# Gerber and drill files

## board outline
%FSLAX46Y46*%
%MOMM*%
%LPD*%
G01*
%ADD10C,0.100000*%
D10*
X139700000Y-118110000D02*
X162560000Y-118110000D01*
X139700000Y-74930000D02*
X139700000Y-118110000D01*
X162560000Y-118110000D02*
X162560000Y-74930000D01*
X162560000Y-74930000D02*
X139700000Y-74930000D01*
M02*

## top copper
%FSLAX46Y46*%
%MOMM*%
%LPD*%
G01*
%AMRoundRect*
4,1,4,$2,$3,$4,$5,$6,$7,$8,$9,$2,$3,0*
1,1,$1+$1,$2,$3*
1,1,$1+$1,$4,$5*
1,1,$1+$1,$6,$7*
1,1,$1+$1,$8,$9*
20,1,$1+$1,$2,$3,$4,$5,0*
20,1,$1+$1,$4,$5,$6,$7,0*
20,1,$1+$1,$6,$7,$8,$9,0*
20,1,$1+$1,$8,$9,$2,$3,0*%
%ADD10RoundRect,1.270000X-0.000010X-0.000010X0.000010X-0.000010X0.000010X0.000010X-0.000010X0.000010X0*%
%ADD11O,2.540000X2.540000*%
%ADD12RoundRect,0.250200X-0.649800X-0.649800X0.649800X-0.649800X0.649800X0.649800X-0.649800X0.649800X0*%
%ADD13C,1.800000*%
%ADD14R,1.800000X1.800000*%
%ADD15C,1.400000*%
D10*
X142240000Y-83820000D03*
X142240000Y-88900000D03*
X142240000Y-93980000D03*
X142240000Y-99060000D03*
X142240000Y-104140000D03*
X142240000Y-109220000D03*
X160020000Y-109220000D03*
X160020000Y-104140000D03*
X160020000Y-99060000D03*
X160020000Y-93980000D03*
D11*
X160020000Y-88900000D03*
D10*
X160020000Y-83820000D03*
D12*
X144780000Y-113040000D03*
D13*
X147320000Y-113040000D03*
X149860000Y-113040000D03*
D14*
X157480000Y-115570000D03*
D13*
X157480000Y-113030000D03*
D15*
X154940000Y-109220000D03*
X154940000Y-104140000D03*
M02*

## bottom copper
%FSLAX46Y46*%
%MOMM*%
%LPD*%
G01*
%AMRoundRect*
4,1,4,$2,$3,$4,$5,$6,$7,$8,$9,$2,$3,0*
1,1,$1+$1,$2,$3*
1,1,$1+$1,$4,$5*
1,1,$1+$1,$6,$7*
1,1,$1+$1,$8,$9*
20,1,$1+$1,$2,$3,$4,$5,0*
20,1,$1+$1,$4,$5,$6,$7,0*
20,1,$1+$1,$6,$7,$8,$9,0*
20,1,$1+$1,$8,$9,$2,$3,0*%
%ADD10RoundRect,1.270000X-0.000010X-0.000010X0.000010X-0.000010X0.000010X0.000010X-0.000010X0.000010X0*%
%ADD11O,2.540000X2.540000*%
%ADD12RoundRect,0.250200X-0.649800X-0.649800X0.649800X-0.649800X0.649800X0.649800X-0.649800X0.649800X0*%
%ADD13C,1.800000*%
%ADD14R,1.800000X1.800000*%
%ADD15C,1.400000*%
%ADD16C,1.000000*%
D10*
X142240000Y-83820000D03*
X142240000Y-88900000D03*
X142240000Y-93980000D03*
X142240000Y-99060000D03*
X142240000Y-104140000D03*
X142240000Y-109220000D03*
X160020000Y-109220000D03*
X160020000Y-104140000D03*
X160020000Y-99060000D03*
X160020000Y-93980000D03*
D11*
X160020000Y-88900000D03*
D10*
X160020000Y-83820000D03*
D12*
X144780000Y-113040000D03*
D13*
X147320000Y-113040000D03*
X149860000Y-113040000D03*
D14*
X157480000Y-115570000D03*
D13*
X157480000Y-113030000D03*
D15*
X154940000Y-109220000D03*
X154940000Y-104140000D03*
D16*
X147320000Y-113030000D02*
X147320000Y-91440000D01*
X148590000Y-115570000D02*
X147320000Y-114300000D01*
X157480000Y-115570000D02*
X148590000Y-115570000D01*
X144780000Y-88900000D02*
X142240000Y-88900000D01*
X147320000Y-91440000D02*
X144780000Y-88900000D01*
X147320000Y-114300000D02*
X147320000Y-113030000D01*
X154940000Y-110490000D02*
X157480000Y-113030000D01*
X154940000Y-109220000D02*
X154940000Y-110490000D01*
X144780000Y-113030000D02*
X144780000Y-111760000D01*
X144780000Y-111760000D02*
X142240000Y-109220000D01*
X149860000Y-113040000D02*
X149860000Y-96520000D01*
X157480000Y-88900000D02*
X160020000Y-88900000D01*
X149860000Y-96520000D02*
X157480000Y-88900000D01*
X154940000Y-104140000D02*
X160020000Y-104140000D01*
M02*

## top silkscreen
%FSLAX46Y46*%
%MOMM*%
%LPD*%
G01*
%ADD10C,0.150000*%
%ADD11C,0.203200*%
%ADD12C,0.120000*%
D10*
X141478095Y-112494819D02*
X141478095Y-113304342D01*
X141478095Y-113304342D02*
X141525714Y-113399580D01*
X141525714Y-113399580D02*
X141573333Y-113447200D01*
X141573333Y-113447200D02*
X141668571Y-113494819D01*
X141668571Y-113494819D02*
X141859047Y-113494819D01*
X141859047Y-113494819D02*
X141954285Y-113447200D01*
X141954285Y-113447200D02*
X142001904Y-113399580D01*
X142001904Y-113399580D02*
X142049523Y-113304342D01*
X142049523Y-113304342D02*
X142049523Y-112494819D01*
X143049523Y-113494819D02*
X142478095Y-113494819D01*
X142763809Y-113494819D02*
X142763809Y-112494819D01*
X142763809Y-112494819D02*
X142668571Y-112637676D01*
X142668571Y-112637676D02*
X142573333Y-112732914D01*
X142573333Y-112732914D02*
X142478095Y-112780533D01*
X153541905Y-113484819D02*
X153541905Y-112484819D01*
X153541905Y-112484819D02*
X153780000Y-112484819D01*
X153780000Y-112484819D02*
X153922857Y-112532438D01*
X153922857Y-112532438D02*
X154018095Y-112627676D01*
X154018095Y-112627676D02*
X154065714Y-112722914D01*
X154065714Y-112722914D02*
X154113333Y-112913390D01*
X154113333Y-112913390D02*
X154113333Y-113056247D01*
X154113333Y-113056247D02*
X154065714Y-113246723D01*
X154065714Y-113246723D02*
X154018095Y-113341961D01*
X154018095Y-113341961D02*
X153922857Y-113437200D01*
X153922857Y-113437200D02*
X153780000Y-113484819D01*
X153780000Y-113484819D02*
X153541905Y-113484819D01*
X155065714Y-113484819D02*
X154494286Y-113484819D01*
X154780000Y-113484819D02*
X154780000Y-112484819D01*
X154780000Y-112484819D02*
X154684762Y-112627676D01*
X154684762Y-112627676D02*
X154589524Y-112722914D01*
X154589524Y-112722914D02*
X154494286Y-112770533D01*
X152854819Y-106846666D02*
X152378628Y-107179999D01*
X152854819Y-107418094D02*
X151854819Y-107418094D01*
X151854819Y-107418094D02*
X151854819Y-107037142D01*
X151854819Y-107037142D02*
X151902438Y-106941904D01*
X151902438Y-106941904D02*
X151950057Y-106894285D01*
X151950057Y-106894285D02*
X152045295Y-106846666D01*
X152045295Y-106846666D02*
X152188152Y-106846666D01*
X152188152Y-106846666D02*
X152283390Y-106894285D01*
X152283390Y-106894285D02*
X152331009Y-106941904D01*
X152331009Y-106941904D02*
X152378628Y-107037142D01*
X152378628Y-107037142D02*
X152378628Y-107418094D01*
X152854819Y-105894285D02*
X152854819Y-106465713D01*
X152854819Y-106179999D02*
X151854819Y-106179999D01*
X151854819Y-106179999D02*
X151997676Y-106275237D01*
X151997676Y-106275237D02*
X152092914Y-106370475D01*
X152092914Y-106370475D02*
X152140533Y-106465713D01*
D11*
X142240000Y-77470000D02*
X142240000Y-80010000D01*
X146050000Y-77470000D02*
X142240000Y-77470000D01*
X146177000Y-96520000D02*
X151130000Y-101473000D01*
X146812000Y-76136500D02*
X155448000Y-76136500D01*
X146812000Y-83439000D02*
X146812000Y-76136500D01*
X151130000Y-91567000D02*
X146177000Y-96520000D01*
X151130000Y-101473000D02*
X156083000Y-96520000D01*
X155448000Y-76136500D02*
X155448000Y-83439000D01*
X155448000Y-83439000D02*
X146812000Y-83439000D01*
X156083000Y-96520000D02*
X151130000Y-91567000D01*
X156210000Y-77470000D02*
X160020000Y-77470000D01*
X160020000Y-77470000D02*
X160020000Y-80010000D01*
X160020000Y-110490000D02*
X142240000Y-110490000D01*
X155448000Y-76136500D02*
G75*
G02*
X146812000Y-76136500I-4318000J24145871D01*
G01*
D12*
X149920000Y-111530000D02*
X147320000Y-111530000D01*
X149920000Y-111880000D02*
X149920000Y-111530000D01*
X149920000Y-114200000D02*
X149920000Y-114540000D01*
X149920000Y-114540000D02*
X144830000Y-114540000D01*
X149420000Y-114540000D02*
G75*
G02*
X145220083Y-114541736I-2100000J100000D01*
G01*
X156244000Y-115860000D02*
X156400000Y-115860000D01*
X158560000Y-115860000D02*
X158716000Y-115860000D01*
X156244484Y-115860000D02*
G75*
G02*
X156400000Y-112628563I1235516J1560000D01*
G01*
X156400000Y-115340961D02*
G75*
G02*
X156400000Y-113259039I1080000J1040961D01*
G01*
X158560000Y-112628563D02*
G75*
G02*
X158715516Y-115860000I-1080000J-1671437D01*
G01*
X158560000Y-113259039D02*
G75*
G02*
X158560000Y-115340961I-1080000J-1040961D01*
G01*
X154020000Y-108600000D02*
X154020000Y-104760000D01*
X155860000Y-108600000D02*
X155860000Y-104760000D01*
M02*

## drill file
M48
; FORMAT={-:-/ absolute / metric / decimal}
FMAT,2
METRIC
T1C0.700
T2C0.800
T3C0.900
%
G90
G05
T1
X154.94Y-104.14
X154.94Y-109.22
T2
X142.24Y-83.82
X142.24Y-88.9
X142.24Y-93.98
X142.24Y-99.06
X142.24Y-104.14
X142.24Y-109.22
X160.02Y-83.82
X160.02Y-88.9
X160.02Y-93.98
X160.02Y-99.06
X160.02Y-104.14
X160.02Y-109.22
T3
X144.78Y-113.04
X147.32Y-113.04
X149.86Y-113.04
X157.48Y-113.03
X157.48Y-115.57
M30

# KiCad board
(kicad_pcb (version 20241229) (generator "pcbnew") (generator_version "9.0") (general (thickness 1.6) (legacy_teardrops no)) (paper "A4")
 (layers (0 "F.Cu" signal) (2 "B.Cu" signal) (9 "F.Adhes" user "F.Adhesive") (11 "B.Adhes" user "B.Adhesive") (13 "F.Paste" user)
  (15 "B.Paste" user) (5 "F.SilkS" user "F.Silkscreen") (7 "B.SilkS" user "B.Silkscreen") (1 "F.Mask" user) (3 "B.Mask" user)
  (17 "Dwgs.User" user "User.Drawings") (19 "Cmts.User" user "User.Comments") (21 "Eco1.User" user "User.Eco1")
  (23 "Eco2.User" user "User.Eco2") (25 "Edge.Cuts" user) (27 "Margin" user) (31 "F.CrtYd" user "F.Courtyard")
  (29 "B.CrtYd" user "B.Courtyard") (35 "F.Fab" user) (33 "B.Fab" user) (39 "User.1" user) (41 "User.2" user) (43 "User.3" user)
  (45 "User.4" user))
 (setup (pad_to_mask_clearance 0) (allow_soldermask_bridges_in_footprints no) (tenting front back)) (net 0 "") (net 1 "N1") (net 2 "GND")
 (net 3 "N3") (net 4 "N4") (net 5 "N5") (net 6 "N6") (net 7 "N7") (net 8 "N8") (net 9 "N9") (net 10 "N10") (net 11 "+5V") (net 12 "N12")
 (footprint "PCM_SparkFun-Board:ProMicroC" (layer "F.Cu") (at 151.13 93.98)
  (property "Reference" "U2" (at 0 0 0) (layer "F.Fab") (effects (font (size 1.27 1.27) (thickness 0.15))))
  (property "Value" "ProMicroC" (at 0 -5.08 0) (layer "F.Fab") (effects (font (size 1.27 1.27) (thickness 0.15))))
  (fp_line (start -8.89 -16.51) (end -8.89 -13.97) (stroke (width 0.2032) (type solid)) (layer "F.SilkS"))
  (fp_line (start -5.08 -16.51) (end -8.89 -16.51) (stroke (width 0.2032) (type solid)) (layer "F.SilkS"))
  (fp_line (start -4.953 2.54) (end 0 7.493) (stroke (width 0.2032) (type solid)) (layer "F.SilkS"))
  (fp_line (start -4.318 -17.8435) (end 4.318 -17.8435) (stroke (width 0.2032) (type solid)) (layer "F.SilkS"))
  (fp_line (start -4.318 -10.541) (end -4.318 -17.8435) (stroke (width 0.2032) (type solid)) (layer "F.SilkS"))
  (fp_line (start 0 -2.413) (end -4.953 2.54) (stroke (width 0.2032) (type solid)) (layer "F.SilkS"))
  (fp_line (start 0 7.493) (end 4.953 2.54) (stroke (width 0.2032) (type solid)) (layer "F.SilkS"))
  (fp_line (start 4.318 -17.8435) (end 4.318 -10.541) (stroke (width 0.2032) (type solid)) (layer "F.SilkS"))
  (fp_line (start 4.318 -10.541) (end -4.318 -10.541) (stroke (width 0.2032) (type solid)) (layer "F.SilkS"))
  (fp_line (start 4.953 2.54) (end 0 -2.413) (stroke (width 0.2032) (type solid)) (layer "F.SilkS"))
  (fp_line (start 5.08 -16.51) (end 8.89 -16.51) (stroke (width 0.2032) (type solid)) (layer "F.SilkS"))
  (fp_line (start 8.89 -16.51) (end 8.89 -13.97) (stroke (width 0.2032) (type solid)) (layer "F.SilkS"))
  (fp_line (start 8.89 16.51) (end -8.89 16.51) (stroke (width 0.2032) (type solid)) (layer "F.SilkS"))
  (fp_arc (start 4.318 -17.8435) (mid 0 -17.460445) (end -4.318 -17.8435) (stroke (width 0.2032) (type solid)) (layer "F.SilkS"))
  (pad "2" thru_hole roundrect (at -8.89 -10.16) (size 2.54 2.54) (drill 0.8) (layers "*.Cu" "*.Mask") (remove_unused_layers no)
   (roundrect_rratio 0.5) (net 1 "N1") (thermal_bridge_angle 0))
  (pad "4" thru_hole roundrect (at -8.89 -5.08) (size 2.54 2.54) (drill 0.8) (layers "*.Cu" "*.Mask") (remove_unused_layers no)
   (roundrect_rratio 0.5) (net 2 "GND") (thermal_bridge_angle 0))
  (pad "6" thru_hole roundrect (at -8.89 0) (size 2.54 2.54) (drill 0.8) (layers "*.Cu" "*.Mask") (remove_unused_layers no)
   (roundrect_rratio 0.5) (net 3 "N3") (thermal_bridge_angle 0))
  (pad "8" thru_hole roundrect (at -8.89 5.08) (size 2.54 2.54) (drill 0.8) (layers "*.Cu" "*.Mask") (remove_unused_layers no)
   (roundrect_rratio 0.5) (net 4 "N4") (thermal_bridge_angle 0))
  (pad "10" thru_hole roundrect (at -8.89 10.16) (size 2.54 2.54) (drill 0.8) (layers "*.Cu" "*.Mask") (remove_unused_layers no)
   (roundrect_rratio 0.5) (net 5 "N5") (thermal_bridge_angle 0))
  (pad "12" thru_hole roundrect (at -8.89 15.24) (size 2.54 2.54) (drill 0.8) (layers "*.Cu" "*.Mask") (remove_unused_layers no)
   (roundrect_rratio 0.5) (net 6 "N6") (thermal_bridge_angle 0))
  (pad "13" thru_hole roundrect (at 8.89 15.24) (size 2.54 2.54) (drill 0.8) (layers "*.Cu" "*.Mask") (remove_unused_layers no)
   (roundrect_rratio 0.5) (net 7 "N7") (thermal_bridge_angle 0))
  (pad "15" thru_hole roundrect (at 8.89 10.16) (size 2.54 2.54) (drill 0.8) (layers "*.Cu" "*.Mask") (remove_unused_layers no)
   (roundrect_rratio 0.5) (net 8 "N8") (thermal_bridge_angle 0))
  (pad "17" thru_hole roundrect (at 8.89 5.08) (size 2.54 2.54) (drill 0.8) (layers "*.Cu" "*.Mask") (remove_unused_layers no)
   (roundrect_rratio 0.5) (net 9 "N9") (thermal_bridge_angle 0))
  (pad "19" thru_hole roundrect (at 8.89 0) (size 2.54 2.54) (drill 0.8) (layers "*.Cu" "*.Mask") (remove_unused_layers no)
   (roundrect_rratio 0.5) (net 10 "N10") (thermal_bridge_angle 0))
  (pad "21" thru_hole oval (at 8.89 -5.08) (size 2.54 2.54) (drill 0.8) (layers "*.Cu" "*.Mask") (remove_unused_layers no) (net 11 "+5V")
   (thermal_bridge_angle 0))
  (pad "23" thru_hole roundrect (at 8.89 -10.16) (size 2.54 2.54) (drill 0.8) (layers "*.Cu" "*.Mask") (remove_unused_layers no)
   (roundrect_rratio 0.5) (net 2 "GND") (thermal_bridge_angle 0)))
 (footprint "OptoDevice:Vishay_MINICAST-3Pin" (layer "F.Cu") (at 144.78 113.04)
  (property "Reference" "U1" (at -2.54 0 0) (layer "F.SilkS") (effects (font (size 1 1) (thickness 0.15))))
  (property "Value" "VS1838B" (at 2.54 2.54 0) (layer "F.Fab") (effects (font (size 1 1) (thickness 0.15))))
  (fp_line (start 5.14 -1.51) (end 2.54 -1.51) (stroke (width 0.12) (type solid)) (layer "F.SilkS"))
  (fp_line (start 5.14 -1.16) (end 5.14 -1.51) (stroke (width 0.12) (type solid)) (layer "F.SilkS"))
  (fp_line (start 5.14 1.16) (end 5.14 1.5) (stroke (width 0.12) (type solid)) (layer "F.SilkS"))
  (fp_line (start 5.14 1.5) (end 0.05 1.5) (stroke (width 0.12) (type solid)) (layer "F.SilkS"))
  (fp_arc (start 4.64 1.5) (mid 2.540869 3.502379) (end 0.440083 1.501736) (stroke (width 0.12) (type solid)) (layer "F.SilkS"))
  (pad "1" thru_hole roundrect (at 0 0) (size 1.8 1.8) (drill 0.9) (layers "*.Cu" "*.Mask") (remove_unused_layers no)
   (roundrect_rratio 0.139))
  (pad "2" thru_hole circle (at 2.54 0) (size 1.8 1.8) (drill 0.9) (layers "*.Cu" "*.Mask") (remove_unused_layers no))
  (pad "3" thru_hole circle (at 5.08 0) (size 1.8 1.8) (drill 0.9) (layers "*.Cu" "*.Mask") (remove_unused_layers no)))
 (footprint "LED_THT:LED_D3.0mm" (layer "F.Cu") (at 157.48 115.57 90)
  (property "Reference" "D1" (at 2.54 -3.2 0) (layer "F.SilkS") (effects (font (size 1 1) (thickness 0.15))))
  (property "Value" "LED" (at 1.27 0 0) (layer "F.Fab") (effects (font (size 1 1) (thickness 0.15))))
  (fp_line (start -0.29 -1.236) (end -0.29 -1.08) (stroke (width 0.12) (type solid)) (layer "F.SilkS"))
  (fp_line (start -0.29 1.08) (end -0.29 1.236) (stroke (width 0.12) (type solid)) (layer "F.SilkS"))
  (fp_arc (start -0.29 -1.235516) (mid 1.36566 -1.987699) (end 2.941437 -1.08) (stroke (width 0.12) (type solid)) (layer "F.SilkS"))
  (fp_arc (start 0.229039 -1.08) (mid 1.27 -1.5) (end 2.310961 -1.08) (stroke (width 0.12) (type solid)) (layer "F.SilkS"))
  (fp_arc (start 2.941437 1.08) (mid 1.36566 1.987699) (end -0.29 1.235516) (stroke (width 0.12) (type solid)) (layer "F.SilkS"))
  (fp_arc (start 2.310961 1.08) (mid 1.27 1.5) (end 0.229039 1.08) (stroke (width 0.12) (type solid)) (layer "F.SilkS"))
  (pad "1" thru_hole rect (at 0 0 90) (size 1.8 1.8) (drill 0.9) (layers "*.Cu" "*.Mask") (remove_unused_layers no) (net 2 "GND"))
  (pad "2" thru_hole circle (at 2.54 0 90) (size 1.8 1.8) (drill 0.9) (layers "*.Cu" "*.Mask") (remove_unused_layers no) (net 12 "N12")))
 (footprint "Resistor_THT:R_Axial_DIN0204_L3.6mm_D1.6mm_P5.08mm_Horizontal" (layer "F.Cu") (at 154.94 109.22 90)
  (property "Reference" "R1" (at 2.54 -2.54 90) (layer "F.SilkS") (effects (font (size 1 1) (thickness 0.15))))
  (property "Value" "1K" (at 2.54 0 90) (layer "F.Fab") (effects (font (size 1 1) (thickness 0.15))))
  (fp_line (start 0.62 -0.92) (end 4.46 -0.92) (stroke (width 0.12) (type solid)) (layer "F.SilkS"))
  (fp_line (start 0.62 0.92) (end 4.46 0.92) (stroke (width 0.12) (type solid)) (layer "F.SilkS"))
  (pad "1" thru_hole circle (at 0 0 90) (size 1.4 1.4) (drill 0.7) (layers "*.Cu" "*.Mask") (remove_unused_layers no) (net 12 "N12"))
  (pad "2" thru_hole circle (at 5.08 0 90) (size 1.4 1.4) (drill 0.7) (layers "*.Cu" "*.Mask") (remove_unused_layers no) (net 8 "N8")))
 (gr_line (start 139.7 118.11) (end 162.56 118.11) (stroke (width 0.1) (type solid)) (layer "Edge.Cuts"))
 (gr_line (start 139.7 74.93) (end 139.7 118.11) (stroke (width 0.1) (type default)) (layer "Edge.Cuts"))
 (gr_line (start 162.56 118.11) (end 162.56 74.93) (stroke (width 0.1) (type default)) (layer "Edge.Cuts"))
 (gr_line (start 162.56 74.93) (end 139.7 74.93) (stroke (width 0.1) (type solid)) (layer "Edge.Cuts"))
 (segment (start 147.32 113.03) (end 147.32 91.44) (width 1) (layer "B.Cu") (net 2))
 (segment (start 148.59 115.57) (end 147.32 114.3) (width 1) (layer "B.Cu") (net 2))
 (segment (start 157.48 115.57) (end 148.59 115.57) (width 1) (layer "B.Cu") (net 2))
 (segment (start 144.78 88.9) (end 142.24 88.9) (width 1) (layer "B.Cu") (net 2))
 (segment (start 147.32 91.44) (end 144.78 88.9) (width 1) (layer "B.Cu") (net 2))
 (segment (start 147.32 114.3) (end 147.32 113.03) (width 1) (layer "B.Cu") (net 2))
 (segment (start 154.94 110.49) (end 157.48 113.03) (width 1) (layer "B.Cu") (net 12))
 (segment (start 154.94 109.22) (end 154.94 110.49) (width 1) (layer "B.Cu") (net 12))
 (segment (start 144.78 113.03) (end 144.78 111.76) (width 1) (layer "B.Cu") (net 6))
 (segment (start 144.78 111.76) (end 142.24 109.22) (width 1) (layer "B.Cu") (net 6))
 (segment (start 149.86 113.04) (end 149.86 96.52) (width 1) (layer "B.Cu") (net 11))
 (segment (start 157.48 88.9) (end 160.02 88.9) (width 1) (layer "B.Cu") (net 11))
 (segment (start 149.86 96.52) (end 157.48 88.9) (width 1) (layer "B.Cu") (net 11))
 (segment (start 154.94 104.14) (end 160.02 104.14) (width 1) (layer "B.Cu") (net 8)))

